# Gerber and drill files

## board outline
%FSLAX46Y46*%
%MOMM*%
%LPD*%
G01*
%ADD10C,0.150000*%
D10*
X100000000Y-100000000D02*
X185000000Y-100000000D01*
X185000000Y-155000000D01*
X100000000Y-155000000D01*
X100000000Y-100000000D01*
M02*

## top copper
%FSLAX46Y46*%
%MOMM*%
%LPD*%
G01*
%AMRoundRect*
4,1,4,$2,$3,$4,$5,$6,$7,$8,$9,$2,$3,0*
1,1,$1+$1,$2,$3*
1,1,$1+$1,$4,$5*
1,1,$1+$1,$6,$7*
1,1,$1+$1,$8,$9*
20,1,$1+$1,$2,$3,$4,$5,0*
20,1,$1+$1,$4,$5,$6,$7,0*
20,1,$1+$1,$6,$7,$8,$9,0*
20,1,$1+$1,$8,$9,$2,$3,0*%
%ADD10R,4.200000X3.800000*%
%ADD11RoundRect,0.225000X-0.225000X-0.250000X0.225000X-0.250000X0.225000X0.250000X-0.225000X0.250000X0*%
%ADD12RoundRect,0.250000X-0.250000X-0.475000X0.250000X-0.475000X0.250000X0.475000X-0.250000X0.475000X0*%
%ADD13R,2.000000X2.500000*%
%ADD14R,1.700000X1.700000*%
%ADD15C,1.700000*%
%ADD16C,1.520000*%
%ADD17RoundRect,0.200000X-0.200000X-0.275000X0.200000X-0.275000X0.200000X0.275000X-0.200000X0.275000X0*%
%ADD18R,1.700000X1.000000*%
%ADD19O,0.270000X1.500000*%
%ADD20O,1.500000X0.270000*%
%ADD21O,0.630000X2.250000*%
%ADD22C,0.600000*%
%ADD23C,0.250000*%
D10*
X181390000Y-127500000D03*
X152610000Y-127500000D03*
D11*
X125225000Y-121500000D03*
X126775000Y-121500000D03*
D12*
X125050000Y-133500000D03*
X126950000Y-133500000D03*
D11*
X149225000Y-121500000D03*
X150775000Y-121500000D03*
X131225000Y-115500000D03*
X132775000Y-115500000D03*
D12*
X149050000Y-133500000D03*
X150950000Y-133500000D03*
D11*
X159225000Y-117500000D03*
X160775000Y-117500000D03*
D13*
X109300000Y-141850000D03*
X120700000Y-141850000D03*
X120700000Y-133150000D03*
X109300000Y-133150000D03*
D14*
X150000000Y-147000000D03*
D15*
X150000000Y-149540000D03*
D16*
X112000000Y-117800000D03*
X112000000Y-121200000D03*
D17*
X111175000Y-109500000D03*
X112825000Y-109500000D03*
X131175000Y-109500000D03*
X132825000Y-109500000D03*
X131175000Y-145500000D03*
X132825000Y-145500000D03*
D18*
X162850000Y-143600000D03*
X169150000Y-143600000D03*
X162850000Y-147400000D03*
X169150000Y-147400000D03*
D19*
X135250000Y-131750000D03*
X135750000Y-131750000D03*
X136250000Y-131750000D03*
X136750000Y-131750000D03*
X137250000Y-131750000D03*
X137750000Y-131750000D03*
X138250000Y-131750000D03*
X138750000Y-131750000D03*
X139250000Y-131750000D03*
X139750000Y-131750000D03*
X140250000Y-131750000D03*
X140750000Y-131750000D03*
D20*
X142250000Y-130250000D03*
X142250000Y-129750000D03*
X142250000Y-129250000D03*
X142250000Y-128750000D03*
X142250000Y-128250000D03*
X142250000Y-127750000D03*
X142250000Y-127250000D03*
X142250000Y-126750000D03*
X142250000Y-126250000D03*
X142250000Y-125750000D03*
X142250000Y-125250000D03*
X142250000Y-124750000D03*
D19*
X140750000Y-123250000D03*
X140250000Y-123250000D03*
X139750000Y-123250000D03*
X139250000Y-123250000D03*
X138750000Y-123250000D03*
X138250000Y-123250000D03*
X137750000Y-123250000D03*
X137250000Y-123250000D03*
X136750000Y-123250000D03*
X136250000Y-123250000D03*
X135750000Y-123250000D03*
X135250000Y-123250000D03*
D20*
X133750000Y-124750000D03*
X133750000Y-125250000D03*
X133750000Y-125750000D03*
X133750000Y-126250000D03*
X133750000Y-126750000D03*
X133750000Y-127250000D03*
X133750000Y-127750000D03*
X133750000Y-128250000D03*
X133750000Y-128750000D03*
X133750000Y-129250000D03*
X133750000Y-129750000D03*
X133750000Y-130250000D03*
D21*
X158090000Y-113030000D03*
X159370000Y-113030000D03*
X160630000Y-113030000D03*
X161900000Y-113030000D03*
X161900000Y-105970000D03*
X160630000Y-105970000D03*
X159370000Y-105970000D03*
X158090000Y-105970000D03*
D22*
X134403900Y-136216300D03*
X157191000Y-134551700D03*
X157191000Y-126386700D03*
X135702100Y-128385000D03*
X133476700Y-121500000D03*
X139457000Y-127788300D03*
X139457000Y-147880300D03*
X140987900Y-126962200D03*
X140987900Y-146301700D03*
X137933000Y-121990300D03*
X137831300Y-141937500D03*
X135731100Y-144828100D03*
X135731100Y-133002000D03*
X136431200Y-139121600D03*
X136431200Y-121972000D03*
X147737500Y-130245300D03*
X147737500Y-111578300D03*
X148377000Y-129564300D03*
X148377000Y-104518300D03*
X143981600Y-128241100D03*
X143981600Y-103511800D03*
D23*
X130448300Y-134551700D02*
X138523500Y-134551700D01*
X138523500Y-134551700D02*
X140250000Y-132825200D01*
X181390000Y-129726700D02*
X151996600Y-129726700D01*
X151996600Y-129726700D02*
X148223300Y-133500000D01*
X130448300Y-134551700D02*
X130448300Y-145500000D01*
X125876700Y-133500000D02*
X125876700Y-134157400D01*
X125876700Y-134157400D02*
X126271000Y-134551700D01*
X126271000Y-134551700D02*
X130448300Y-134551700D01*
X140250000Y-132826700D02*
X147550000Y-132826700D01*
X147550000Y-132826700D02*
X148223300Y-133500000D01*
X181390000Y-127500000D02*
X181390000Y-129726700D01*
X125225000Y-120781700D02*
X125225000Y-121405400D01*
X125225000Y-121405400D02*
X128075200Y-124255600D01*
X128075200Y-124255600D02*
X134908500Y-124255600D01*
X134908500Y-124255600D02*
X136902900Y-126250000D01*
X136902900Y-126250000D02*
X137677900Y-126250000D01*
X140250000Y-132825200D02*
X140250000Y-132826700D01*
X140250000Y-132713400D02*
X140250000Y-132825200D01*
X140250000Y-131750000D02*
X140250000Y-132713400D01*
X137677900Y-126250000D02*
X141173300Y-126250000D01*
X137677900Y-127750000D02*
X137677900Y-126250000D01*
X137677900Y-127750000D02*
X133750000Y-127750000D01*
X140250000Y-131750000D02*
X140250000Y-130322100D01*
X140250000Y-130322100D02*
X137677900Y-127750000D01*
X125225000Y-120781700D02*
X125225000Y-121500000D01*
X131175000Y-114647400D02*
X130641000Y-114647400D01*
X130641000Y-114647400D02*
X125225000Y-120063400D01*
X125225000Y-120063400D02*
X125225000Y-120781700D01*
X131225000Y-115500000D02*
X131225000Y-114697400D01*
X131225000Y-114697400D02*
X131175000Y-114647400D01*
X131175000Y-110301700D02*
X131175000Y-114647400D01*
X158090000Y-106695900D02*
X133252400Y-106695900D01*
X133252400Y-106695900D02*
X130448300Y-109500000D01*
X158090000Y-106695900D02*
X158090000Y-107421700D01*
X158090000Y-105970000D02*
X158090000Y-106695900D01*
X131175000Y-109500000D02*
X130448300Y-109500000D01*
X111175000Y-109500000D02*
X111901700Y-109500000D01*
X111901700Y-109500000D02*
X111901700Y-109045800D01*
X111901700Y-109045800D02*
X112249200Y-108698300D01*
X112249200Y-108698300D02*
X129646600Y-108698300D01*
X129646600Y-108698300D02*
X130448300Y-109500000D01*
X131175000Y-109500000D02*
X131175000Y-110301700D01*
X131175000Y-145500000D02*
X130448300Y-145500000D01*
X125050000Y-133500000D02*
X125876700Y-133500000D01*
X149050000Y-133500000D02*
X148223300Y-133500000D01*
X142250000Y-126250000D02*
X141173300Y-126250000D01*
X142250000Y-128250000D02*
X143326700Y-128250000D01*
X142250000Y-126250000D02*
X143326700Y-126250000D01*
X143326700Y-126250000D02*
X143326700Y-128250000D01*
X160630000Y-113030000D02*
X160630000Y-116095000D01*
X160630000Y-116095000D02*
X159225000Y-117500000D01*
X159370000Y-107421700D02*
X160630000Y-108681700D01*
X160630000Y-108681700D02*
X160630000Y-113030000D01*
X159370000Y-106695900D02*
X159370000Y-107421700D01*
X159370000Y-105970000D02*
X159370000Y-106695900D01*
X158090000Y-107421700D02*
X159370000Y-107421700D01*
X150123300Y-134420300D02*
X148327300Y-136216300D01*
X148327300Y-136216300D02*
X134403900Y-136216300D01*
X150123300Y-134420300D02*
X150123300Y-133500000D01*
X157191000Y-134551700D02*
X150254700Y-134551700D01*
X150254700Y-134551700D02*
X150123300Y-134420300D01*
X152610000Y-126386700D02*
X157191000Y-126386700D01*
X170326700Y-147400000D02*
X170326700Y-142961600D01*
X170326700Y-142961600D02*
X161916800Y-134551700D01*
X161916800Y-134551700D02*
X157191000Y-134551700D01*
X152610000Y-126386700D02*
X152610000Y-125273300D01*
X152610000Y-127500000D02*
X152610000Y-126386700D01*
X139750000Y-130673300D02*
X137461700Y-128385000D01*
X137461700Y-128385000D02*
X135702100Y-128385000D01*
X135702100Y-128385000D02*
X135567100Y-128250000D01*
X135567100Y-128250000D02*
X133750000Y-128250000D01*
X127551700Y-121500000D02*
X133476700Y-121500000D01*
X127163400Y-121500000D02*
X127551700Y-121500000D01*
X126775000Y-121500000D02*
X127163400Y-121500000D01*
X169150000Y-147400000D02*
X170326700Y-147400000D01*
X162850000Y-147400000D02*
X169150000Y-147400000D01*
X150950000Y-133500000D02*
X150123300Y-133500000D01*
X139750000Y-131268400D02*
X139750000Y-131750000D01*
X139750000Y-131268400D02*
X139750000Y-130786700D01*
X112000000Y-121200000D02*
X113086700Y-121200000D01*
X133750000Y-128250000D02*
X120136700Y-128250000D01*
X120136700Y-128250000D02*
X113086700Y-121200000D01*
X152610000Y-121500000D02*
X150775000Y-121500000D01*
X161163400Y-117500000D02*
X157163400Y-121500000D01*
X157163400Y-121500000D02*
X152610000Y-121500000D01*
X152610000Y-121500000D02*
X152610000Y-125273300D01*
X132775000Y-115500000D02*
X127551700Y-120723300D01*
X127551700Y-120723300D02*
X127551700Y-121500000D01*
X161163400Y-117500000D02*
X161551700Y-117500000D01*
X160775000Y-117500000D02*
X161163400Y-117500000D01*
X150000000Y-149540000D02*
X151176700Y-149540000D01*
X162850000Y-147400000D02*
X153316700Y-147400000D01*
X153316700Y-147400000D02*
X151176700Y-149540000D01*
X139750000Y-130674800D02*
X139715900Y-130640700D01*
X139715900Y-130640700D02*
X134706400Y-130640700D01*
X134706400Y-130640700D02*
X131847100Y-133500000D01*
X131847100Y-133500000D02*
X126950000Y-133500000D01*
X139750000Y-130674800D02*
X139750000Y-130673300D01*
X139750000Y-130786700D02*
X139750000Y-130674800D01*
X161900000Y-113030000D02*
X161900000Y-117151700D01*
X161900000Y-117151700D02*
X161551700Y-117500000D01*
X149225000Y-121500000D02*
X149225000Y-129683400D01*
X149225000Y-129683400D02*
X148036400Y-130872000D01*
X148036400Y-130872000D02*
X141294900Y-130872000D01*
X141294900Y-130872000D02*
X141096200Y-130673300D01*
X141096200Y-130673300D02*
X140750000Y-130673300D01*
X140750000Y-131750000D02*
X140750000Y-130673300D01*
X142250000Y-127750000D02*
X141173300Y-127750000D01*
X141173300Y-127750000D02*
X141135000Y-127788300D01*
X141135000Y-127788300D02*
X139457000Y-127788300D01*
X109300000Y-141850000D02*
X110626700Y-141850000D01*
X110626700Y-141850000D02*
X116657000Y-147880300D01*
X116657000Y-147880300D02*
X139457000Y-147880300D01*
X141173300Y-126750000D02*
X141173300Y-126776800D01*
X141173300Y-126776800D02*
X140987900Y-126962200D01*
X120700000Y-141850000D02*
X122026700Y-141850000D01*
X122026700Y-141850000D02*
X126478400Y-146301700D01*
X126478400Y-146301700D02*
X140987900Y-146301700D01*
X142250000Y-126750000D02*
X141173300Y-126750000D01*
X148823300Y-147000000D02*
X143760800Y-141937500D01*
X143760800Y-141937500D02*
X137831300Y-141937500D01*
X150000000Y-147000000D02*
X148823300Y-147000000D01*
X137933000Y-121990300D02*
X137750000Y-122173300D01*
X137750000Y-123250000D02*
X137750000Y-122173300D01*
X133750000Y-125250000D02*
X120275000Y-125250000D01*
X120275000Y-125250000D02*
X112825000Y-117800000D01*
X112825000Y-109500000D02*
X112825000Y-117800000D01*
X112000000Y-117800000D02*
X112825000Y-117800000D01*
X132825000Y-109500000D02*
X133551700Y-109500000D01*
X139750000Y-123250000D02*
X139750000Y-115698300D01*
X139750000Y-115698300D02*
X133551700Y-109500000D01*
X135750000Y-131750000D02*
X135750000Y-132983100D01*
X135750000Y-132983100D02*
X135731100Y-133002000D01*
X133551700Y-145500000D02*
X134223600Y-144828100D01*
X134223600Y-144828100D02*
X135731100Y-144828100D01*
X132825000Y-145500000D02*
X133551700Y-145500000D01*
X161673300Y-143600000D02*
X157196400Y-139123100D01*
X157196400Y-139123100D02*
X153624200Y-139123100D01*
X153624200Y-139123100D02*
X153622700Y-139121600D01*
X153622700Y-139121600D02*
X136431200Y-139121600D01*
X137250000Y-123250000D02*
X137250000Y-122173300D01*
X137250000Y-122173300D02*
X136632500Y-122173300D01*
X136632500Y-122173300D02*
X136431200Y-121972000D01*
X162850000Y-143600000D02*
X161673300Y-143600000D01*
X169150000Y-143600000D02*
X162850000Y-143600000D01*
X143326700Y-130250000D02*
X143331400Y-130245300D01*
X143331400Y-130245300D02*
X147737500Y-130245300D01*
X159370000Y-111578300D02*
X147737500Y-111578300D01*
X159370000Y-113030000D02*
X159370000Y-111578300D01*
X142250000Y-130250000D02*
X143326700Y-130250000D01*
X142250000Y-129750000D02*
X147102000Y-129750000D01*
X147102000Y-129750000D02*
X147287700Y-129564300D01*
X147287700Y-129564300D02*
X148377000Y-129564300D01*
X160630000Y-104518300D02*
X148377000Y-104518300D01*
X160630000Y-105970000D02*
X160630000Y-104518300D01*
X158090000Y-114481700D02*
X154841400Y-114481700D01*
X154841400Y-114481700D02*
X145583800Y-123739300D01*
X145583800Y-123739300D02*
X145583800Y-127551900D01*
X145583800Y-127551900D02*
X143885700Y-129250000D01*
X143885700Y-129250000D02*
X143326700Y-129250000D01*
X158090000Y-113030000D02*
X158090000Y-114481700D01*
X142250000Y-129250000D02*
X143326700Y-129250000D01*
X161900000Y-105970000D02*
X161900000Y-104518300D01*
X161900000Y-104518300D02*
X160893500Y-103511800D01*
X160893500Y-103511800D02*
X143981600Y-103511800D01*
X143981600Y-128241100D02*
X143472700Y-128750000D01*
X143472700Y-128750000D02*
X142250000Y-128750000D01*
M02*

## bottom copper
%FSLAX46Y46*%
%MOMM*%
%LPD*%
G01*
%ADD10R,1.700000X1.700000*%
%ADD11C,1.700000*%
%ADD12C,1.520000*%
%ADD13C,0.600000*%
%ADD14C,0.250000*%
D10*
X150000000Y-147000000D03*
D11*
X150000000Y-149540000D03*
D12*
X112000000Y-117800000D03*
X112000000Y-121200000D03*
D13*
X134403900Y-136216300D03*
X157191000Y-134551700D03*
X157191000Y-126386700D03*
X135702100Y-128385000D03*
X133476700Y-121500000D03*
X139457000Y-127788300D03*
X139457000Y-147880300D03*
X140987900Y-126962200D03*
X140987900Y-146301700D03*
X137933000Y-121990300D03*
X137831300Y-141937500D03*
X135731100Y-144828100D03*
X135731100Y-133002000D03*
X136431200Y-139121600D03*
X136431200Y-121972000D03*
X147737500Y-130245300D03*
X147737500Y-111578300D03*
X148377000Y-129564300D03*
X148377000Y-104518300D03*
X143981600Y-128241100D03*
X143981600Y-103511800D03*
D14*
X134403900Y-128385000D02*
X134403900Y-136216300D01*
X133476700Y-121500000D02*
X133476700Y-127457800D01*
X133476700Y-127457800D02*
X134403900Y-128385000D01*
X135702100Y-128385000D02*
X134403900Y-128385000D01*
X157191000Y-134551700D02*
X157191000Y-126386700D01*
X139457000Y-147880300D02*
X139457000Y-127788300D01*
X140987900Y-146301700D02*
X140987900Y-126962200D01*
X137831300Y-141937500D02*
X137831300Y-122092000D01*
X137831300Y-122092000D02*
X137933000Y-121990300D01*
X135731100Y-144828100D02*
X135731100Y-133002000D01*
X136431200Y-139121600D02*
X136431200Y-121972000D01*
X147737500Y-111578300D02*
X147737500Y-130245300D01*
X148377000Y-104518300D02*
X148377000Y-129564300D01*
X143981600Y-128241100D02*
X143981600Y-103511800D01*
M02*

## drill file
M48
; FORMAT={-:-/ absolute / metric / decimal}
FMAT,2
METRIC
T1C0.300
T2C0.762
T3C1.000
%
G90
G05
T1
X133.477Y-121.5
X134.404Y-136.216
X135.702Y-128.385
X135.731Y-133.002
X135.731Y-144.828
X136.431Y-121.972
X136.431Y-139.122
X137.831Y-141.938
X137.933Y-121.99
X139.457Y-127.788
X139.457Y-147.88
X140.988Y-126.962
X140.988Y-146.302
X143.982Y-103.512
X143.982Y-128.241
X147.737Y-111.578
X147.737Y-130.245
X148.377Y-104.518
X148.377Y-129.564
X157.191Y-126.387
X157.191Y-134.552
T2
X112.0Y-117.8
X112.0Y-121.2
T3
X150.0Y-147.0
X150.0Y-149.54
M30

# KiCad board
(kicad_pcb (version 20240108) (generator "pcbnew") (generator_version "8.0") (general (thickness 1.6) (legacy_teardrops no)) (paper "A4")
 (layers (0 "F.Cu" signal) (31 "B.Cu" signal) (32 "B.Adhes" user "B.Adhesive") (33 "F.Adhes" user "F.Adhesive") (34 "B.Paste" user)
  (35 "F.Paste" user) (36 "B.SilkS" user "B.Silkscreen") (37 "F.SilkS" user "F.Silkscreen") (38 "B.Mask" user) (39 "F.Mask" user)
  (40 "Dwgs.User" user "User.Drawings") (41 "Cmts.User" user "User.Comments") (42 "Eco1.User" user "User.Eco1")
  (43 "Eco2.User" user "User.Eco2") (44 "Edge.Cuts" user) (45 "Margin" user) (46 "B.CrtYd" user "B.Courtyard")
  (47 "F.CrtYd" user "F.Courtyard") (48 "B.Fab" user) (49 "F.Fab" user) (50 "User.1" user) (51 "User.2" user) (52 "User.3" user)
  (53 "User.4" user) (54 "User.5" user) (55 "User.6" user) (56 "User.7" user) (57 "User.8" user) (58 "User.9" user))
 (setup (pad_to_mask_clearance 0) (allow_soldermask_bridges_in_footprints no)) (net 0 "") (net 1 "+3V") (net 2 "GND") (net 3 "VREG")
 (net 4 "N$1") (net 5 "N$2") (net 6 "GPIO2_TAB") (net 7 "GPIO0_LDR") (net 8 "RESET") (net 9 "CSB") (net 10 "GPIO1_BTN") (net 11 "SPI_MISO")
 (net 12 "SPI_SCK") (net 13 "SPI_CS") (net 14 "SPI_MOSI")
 (gr_rect (start 100.0 100.0) (end 185.0 155.0) (stroke (width 0.15) (type default)) (fill none) (layer "Edge.Cuts"))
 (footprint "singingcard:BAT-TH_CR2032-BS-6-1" (layer "F.Cu") (at 167.0 127.5 0)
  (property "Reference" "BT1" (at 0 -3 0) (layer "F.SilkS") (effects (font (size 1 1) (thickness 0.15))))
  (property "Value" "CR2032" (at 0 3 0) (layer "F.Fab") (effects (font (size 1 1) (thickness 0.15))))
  (pad "1" smd rect (at 14.39 0) (size 4.2 3.8) (layers "F.Cu" "F.Mask" "F.Paste") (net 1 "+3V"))
  (pad "2" smd rect (at -14.39 0) (size 4.2 3.8) (layers "F.Cu" "F.Mask" "F.Paste") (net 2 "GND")))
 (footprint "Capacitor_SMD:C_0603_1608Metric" (layer "F.Cu") (at 126.0 121.5 0)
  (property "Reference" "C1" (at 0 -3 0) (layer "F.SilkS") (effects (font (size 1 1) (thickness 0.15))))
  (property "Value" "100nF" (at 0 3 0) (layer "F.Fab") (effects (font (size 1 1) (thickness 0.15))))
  (pad "1" smd roundrect (at -0.775 0) (size 0.9 0.95) (layers "F.Cu" "F.Mask" "F.Paste") (roundrect_rratio 0.25) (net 1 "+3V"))
  (pad "2" smd roundrect (at 0.775 0) (size 0.9 0.95) (layers "F.Cu" "F.Mask" "F.Paste") (roundrect_rratio 0.25) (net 2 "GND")))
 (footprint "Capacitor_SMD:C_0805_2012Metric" (layer "F.Cu") (at 126.0 133.5 0)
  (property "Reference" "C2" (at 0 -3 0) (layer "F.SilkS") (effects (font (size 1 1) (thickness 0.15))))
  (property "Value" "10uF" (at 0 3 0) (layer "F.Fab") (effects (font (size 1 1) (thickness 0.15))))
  (pad "1" smd roundrect (at -0.95 0) (size 1 1.45) (layers "F.Cu" "F.Mask" "F.Paste") (roundrect_rratio 0.25) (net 1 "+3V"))
  (pad "2" smd roundrect (at 0.95 0) (size 1 1.45) (layers "F.Cu" "F.Mask" "F.Paste") (roundrect_rratio 0.25) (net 2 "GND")))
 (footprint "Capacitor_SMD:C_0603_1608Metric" (layer "F.Cu") (at 150.0 121.5 0)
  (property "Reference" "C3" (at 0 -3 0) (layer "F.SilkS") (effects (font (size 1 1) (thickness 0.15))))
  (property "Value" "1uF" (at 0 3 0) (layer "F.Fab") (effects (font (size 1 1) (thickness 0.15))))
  (pad "1" smd roundrect (at -0.775 0) (size 0.9 0.95) (layers "F.Cu" "F.Mask" "F.Paste") (roundrect_rratio 0.25) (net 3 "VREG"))
  (pad "2" smd roundrect (at 0.775 0) (size 0.9 0.95) (layers "F.Cu" "F.Mask" "F.Paste") (roundrect_rratio 0.25) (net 2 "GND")))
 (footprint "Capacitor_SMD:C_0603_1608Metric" (layer "F.Cu") (at 132.0 115.5 0)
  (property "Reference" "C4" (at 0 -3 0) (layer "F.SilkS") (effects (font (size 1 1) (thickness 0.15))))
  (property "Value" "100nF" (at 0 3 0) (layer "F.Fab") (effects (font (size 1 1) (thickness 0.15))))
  (pad "1" smd roundrect (at -0.775 0) (size 0.9 0.95) (layers "F.Cu" "F.Mask" "F.Paste") (roundrect_rratio 0.25) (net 1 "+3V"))
  (pad "2" smd roundrect (at 0.775 0) (size 0.9 0.95) (layers "F.Cu" "F.Mask" "F.Paste") (roundrect_rratio 0.25) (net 2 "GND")))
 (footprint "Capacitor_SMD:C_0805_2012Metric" (layer "F.Cu") (at 150.0 133.5 0)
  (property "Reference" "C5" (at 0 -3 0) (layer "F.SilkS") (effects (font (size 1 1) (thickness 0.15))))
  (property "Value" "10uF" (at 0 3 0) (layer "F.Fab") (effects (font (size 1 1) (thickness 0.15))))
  (pad "1" smd roundrect (at -0.95 0) (size 1 1.45) (layers "F.Cu" "F.Mask" "F.Paste") (roundrect_rratio 0.25) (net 1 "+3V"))
  (pad "2" smd roundrect (at 0.95 0) (size 1 1.45) (layers "F.Cu" "F.Mask" "F.Paste") (roundrect_rratio 0.25) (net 2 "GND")))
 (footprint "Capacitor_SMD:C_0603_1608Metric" (layer "F.Cu") (at 160.0 117.5 0)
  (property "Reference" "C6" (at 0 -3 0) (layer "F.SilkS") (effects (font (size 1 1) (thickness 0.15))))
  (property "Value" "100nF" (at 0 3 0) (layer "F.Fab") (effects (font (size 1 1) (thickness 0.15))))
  (pad "1" smd roundrect (at -0.775 0) (size 0.9 0.95) (layers "F.Cu" "F.Mask" "F.Paste") (roundrect_rratio 0.25) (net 1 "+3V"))
  (pad "2" smd roundrect (at 0.775 0) (size 0.9 0.95) (layers "F.Cu" "F.Mask" "F.Paste") (roundrect_rratio 0.25) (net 2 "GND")))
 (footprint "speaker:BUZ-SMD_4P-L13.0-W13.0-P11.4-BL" (layer "F.Cu") (at 115.0 137.5 0)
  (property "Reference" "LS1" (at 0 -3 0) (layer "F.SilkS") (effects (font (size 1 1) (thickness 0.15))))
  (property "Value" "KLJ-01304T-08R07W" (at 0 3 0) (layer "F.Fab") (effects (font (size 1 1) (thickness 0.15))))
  (pad "1" smd rect (at -5.7 4.35) (size 2 2.5) (layers "F.Cu" "F.Mask" "F.Paste") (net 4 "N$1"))
  (pad "2" smd rect (at 5.7 4.35) (size 2 2.5) (layers "F.Cu" "F.Mask" "F.Paste") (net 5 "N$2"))
  (pad "3" smd rect (at 5.7 -4.35) (size 2 2.5) (layers "F.Cu" "F.Mask" "F.Paste"))
  (pad "4" smd rect (at -5.7 -4.35) (size 2 2.5) (layers "F.Cu" "F.Mask" "F.Paste")))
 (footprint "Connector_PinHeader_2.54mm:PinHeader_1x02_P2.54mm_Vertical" (layer "F.Cu") (at 150.0 147.0 0)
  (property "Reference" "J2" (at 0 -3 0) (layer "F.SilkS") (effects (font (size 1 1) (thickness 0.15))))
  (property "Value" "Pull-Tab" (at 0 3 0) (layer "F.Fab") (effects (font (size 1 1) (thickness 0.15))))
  (pad "1" thru_hole rect (at 0 0) (size 1.7 1.7) (drill 1) (layers "*.Cu" "*.Mask") (remove_unused_layers no) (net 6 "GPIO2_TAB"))
  (pad "2" thru_hole circle (at 0 2.54) (size 1.7 1.7) (drill 1) (layers "*.Cu" "*.Mask") (remove_unused_layers no) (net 2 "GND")))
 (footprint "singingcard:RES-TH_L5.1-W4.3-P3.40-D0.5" (layer "F.Cu") (at 112.0 119.5 0)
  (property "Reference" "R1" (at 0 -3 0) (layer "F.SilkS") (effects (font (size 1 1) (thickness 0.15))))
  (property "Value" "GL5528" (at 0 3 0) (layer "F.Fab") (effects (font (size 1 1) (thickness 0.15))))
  (pad "1" thru_hole circle (at 0 -1.7 270) (size 1.52 1.52) (drill 0.762) (layers "*.Cu" "*.Mask") (remove_unused_layers no)
   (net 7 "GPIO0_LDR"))
  (pad "2" thru_hole circle (at 0 1.7 270) (size 1.52 1.52) (drill 0.762) (layers "*.Cu" "*.Mask") (remove_unused_layers no) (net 2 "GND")))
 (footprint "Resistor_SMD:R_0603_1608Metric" (layer "F.Cu") (at 112.0 109.5 0)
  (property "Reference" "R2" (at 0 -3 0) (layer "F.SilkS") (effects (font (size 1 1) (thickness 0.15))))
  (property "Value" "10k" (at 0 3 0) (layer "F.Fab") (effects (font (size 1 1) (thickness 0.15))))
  (pad "1" smd roundrect (at -0.825 0) (size 0.8 0.95) (layers "F.Cu" "F.Mask" "F.Paste") (roundrect_rratio 0.25) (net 1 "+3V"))
  (pad "2" smd roundrect (at 0.825 0) (size 0.8 0.95) (layers "F.Cu" "F.Mask" "F.Paste") (roundrect_rratio 0.25) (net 7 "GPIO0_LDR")))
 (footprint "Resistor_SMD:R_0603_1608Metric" (layer "F.Cu") (at 132.0 109.5 0)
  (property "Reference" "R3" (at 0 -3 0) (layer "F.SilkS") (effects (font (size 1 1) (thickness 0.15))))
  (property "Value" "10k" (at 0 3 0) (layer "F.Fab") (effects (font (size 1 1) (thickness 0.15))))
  (pad "1" smd roundrect (at -0.825 0) (size 0.8 0.95) (layers "F.Cu" "F.Mask" "F.Paste") (roundrect_rratio 0.25) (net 1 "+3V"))
  (pad "2" smd roundrect (at 0.825 0) (size 0.8 0.95) (layers "F.Cu" "F.Mask" "F.Paste") (roundrect_rratio 0.25) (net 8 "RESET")))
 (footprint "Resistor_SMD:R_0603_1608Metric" (layer "F.Cu") (at 132.0 145.5 0)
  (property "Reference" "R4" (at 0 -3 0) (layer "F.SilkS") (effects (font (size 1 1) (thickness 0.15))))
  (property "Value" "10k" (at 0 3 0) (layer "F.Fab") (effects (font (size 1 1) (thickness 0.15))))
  (pad "1" smd roundrect (at -0.825 0) (size 0.8 0.95) (layers "F.Cu" "F.Mask" "F.Paste") (roundrect_rratio 0.25) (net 1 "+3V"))
  (pad "2" smd roundrect (at 0.825 0) (size 0.8 0.95) (layers "F.Cu" "F.Mask" "F.Paste") (roundrect_rratio 0.25) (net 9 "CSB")))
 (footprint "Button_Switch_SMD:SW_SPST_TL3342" (layer "F.Cu") (at 166.0 145.5 0)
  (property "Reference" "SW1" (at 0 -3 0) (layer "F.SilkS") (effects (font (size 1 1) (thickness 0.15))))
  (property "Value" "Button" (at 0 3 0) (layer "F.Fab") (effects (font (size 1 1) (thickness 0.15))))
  (pad "1" smd rect (at -3.15 -1.9) (size 1.7 1) (layers "F.Cu" "F.Mask" "F.Paste") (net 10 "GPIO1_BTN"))
  (pad "1" smd rect (at 3.15 -1.9) (size 1.7 1) (layers "F.Cu" "F.Mask" "F.Paste") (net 10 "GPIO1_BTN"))
  (pad "2" smd rect (at -3.15 1.9) (size 1.7 1) (layers "F.Cu" "F.Mask" "F.Paste") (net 2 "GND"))
  (pad "2" smd rect (at 3.15 1.9) (size 1.7 1) (layers "F.Cu" "F.Mask" "F.Paste") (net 2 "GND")))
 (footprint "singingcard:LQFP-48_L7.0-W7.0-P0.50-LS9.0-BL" (layer "F.Cu") (at 138.0 127.5 0)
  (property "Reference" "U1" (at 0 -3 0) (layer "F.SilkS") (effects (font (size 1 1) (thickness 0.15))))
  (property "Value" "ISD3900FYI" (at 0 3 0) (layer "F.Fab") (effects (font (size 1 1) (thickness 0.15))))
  (pad "1" smd oval (at -2.75 4.25) (size 0.27 1.5) (layers "F.Cu" "F.Mask" "F.Paste"))
  (pad "2" smd oval (at -2.25 4.25) (size 0.27 1.5) (layers "F.Cu" "F.Mask" "F.Paste") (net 9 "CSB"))
  (pad "3" smd oval (at -1.75 4.25) (size 0.27 1.5) (layers "F.Cu" "F.Mask" "F.Paste"))
  (pad "4" smd oval (at -1.25 4.25) (size 0.27 1.5) (layers "F.Cu" "F.Mask" "F.Paste"))
  (pad "5" smd oval (at -0.75 4.25) (size 0.27 1.5) (layers "F.Cu" "F.Mask" "F.Paste"))
  (pad "6" smd oval (at -0.25 4.25) (size 0.27 1.5) (layers "F.Cu" "F.Mask" "F.Paste"))
  (pad "7" smd oval (at 0.25 4.25) (size 0.27 1.5) (layers "F.Cu" "F.Mask" "F.Paste"))
  (pad "8" smd oval (at 0.75 4.25) (size 0.27 1.5) (layers "F.Cu" "F.Mask" "F.Paste"))
  (pad "9" smd oval (at 1.25 4.25) (size 0.27 1.5) (layers "F.Cu" "F.Mask" "F.Paste"))
  (pad "10" smd oval (at 1.75 4.25) (size 0.27 1.5) (layers "F.Cu" "F.Mask" "F.Paste") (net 2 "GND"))
  (pad "11" smd oval (at 2.25 4.25) (size 0.27 1.5) (layers "F.Cu" "F.Mask" "F.Paste") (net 1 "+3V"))
  (pad "12" smd oval (at 2.75 4.25) (size 0.27 1.5) (layers "F.Cu" "F.Mask" "F.Paste") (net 3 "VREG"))
  (pad "13" smd oval (at 4.25 2.75) (size 1.5 0.27) (layers "F.Cu" "F.Mask" "F.Paste") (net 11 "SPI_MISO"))
  (pad "14" smd oval (at 4.25 2.25) (size 1.5 0.27) (layers "F.Cu" "F.Mask" "F.Paste") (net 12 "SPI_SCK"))
  (pad "15" smd oval (at 4.25 1.75) (size 1.5 0.27) (layers "F.Cu" "F.Mask" "F.Paste") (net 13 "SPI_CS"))
  (pad "16" smd oval (at 4.25 1.25) (size 1.5 0.27) (layers "F.Cu" "F.Mask" "F.Paste") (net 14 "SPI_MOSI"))
  (pad "17" smd oval (at 4.25 0.75) (size 1.5 0.27) (layers "F.Cu" "F.Mask" "F.Paste") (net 1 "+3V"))
  (pad "18" smd oval (at 4.25 0.25) (size 1.5 0.27) (layers "F.Cu" "F.Mask" "F.Paste") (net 4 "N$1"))
  (pad "19" smd oval (at 4.25 -0.25) (size 1.5 0.27) (layers "F.Cu" "F.Mask" "F.Paste"))
  (pad "20" smd oval (at 4.25 -0.75) (size 1.5 0.27) (layers "F.Cu" "F.Mask" "F.Paste") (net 5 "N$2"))
  (pad "21" smd oval (at 4.25 -1.25) (size 1.5 0.27) (layers "F.Cu" "F.Mask" "F.Paste") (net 1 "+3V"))
  (pad "22" smd oval (at 4.25 -1.75) (size 1.5 0.27) (layers "F.Cu" "F.Mask" "F.Paste"))
  (pad "23" smd oval (at 4.25 -2.25) (size 1.5 0.27) (layers "F.Cu" "F.Mask" "F.Paste"))
  (pad "24" smd oval (at 4.25 -2.75) (size 1.5 0.27) (layers "F.Cu" "F.Mask" "F.Paste"))
  (pad "25" smd oval (at 2.75 -4.25) (size 0.27 1.5) (layers "F.Cu" "F.Mask" "F.Paste"))
  (pad "26" smd oval (at 2.25 -4.25) (size 0.27 1.5) (layers "F.Cu" "F.Mask" "F.Paste"))
  (pad "27" smd oval (at 1.75 -4.25) (size 0.27 1.5) (layers "F.Cu" "F.Mask" "F.Paste") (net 8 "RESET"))
  (pad "28" smd oval (at 1.25 -4.25) (size 0.27 1.5) (layers "F.Cu" "F.Mask" "F.Paste"))
  (pad "29" smd oval (at 0.75 -4.25) (size 0.27 1.5) (layers "F.Cu" "F.Mask" "F.Paste"))
  (pad "30" smd oval (at 0.25 -4.25) (size 0.27 1.5) (layers "F.Cu" "F.Mask" "F.Paste"))
  (pad "31" smd oval (at -0.25 -4.25) (size 0.27 1.5) (layers "F.Cu" "F.Mask" "F.Paste") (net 6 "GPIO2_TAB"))
  (pad "32" smd oval (at -0.75 -4.25) (size 0.27 1.5) (layers "F.Cu" "F.Mask" "F.Paste") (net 10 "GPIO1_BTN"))
  (pad "33" smd oval (at -1.25 -4.25) (size 0.27 1.5) (layers "F.Cu" "F.Mask" "F.Paste"))
  (pad "34" smd oval (at -1.75 -4.25) (size 0.27 1.5) (layers "F.Cu" "F.Mask" "F.Paste"))
  (pad "35" smd oval (at -2.25 -4.25) (size 0.27 1.5) (layers "F.Cu" "F.Mask" "F.Paste"))
  (pad "36" smd oval (at -2.75 -4.25) (size 0.27 1.5) (layers "F.Cu" "F.Mask" "F.Paste"))
  (pad "37" smd oval (at -4.25 -2.75) (size 1.5 0.27) (layers "F.Cu" "F.Mask" "F.Paste"))
  (pad "38" smd oval (at -4.25 -2.25) (size 1.5 0.27) (layers "F.Cu" "F.Mask" "F.Paste") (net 7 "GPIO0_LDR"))
  (pad "39" smd oval (at -4.25 -1.75) (size 1.5 0.27) (layers "F.Cu" "F.Mask" "F.Paste"))
  (pad "40" smd oval (at -4.25 -1.25) (size 1.5 0.27) (layers "F.Cu" "F.Mask" "F.Paste"))
  (pad "41" smd oval (at -4.25 -0.75) (size 1.5 0.27) (layers "F.Cu" "F.Mask" "F.Paste"))
  (pad "42" smd oval (at -4.25 -0.25) (size 1.5 0.27) (layers "F.Cu" "F.Mask" "F.Paste"))
  (pad "43" smd oval (at -4.25 0.25) (size 1.5 0.27) (layers "F.Cu" "F.Mask" "F.Paste") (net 1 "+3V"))
  (pad "44" smd oval (at -4.25 0.75) (size 1.5 0.27) (layers "F.Cu" "F.Mask" "F.Paste") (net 2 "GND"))
  (pad "45" smd oval (at -4.25 1.25) (size 1.5 0.27) (layers "F.Cu" "F.Mask" "F.Paste"))
  (pad "46" smd oval (at -4.25 1.75) (size 1.5 0.27) (layers "F.Cu" "F.Mask" "F.Paste"))
  (pad "47" smd oval (at -4.25 2.25) (size 1.5 0.27) (layers "F.Cu" "F.Mask" "F.Paste"))
  (pad "48" smd oval (at -4.25 2.75) (size 1.5 0.27) (layers "F.Cu" "F.Mask" "F.Paste")))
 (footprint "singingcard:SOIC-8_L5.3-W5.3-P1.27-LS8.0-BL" (layer "F.Cu") (at 160.0 109.5 0)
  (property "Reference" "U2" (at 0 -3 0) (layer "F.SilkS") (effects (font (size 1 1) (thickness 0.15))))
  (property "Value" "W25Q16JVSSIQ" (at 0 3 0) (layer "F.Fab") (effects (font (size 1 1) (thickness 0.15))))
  (pad "1" smd oval (at -1.91 3.53) (size 0.63 2.25) (layers "F.Cu" "F.Mask" "F.Paste") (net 13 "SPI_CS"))
  (pad "2" smd oval (at -0.63 3.53) (size 0.63 2.25) (layers "F.Cu" "F.Mask" "F.Paste") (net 11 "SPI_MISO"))
  (pad "3" smd oval (at 0.63 3.53) (size 0.63 2.25) (layers "F.Cu" "F.Mask" "F.Paste") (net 1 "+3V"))
  (pad "4" smd oval (at 1.9 3.53) (size 0.63 2.25) (layers "F.Cu" "F.Mask" "F.Paste") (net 2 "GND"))
  (pad "5" smd oval (at 1.9 -3.53) (size 0.63 2.25) (layers "F.Cu" "F.Mask" "F.Paste") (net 14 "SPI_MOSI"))
  (pad "6" smd oval (at 0.63 -3.53) (size 0.63 2.25) (layers "F.Cu" "F.Mask" "F.Paste") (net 12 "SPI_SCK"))
  (pad "7" smd oval (at -0.63 -3.53) (size 0.63 2.25) (layers "F.Cu" "F.Mask" "F.Paste") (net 1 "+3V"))
  (pad "8" smd oval (at -1.91 -3.53) (size 0.63 2.25) (layers "F.Cu" "F.Mask" "F.Paste") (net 1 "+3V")))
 (segment (start 130.4483 134.5517) (end 138.5235 134.5517) (width 0.2500) (layer "F.Cu") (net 1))
 (segment (start 138.5235 134.5517) (end 140.2500 132.8252) (width 0.2500) (layer "F.Cu") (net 1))
 (segment (start 181.3900 129.7267) (end 151.9966 129.7267) (width 0.2500) (layer "F.Cu") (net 1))
 (segment (start 151.9966 129.7267) (end 148.2233 133.5000) (width 0.2500) (layer "F.Cu") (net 1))
 (segment (start 130.4483 134.5517) (end 130.4483 145.5000) (width 0.2500) (layer "F.Cu") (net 1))
 (segment (start 125.8767 133.5000) (end 125.8767 134.1574) (width 0.2500) (layer "F.Cu") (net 1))
 (segment (start 125.8767 134.1574) (end 126.2710 134.5517) (width 0.2500) (layer "F.Cu") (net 1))
 (segment (start 126.2710 134.5517) (end 130.4483 134.5517) (width 0.2500) (layer "F.Cu") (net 1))
 (segment (start 140.2500 132.8267) (end 147.5500 132.8267) (width 0.2500) (layer "F.Cu") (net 1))
 (segment (start 147.5500 132.8267) (end 148.2233 133.5000) (width 0.2500) (layer "F.Cu") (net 1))
 (segment (start 181.3900 127.5000) (end 181.3900 129.7267) (width 0.2500) (layer "F.Cu") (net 1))
 (segment (start 125.2250 120.7817) (end 125.2250 121.4054) (width 0.2500) (layer "F.Cu") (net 1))
 (segment (start 125.2250 121.4054) (end 128.0752 124.2556) (width 0.2500) (layer "F.Cu") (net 1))
 (segment (start 128.0752 124.2556) (end 134.9085 124.2556) (width 0.2500) (layer "F.Cu") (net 1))
 (segment (start 134.9085 124.2556) (end 136.9029 126.2500) (width 0.2500) (layer "F.Cu") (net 1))
 (segment (start 136.9029 126.2500) (end 137.6779 126.2500) (width 0.2500) (layer "F.Cu") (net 1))
 (segment (start 140.2500 132.8252) (end 140.2500 132.8267) (width 0.2500) (layer "F.Cu") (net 1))
 (segment (start 140.2500 132.7134) (end 140.2500 132.8252) (width 0.2500) (layer "F.Cu") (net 1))
 (segment (start 140.2500 131.7500) (end 140.2500 132.7134) (width 0.2500) (layer "F.Cu") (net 1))
 (segment (start 137.6779 126.2500) (end 141.1733 126.2500) (width 0.2500) (layer "F.Cu") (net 1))
 (segment (start 137.6779 127.7500) (end 137.6779 126.2500) (width 0.2500) (layer "F.Cu") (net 1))
 (segment (start 137.6779 127.7500) (end 133.7500 127.7500) (width 0.2500) (layer "F.Cu") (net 1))
 (segment (start 140.2500 131.7500) (end 140.2500 130.3221) (width 0.2500) (layer "F.Cu") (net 1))
 (segment (start 140.2500 130.3221) (end 137.6779 127.7500) (width 0.2500) (layer "F.Cu") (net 1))
 (segment (start 125.2250 120.7817) (end 125.2250 121.5000) (width 0.2500) (layer "F.Cu") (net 1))
 (segment (start 131.1750 114.6474) (end 130.6410 114.6474) (width 0.2500) (layer "F.Cu") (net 1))
 (segment (start 130.6410 114.6474) (end 125.2250 120.0634) (width 0.2500) (layer "F.Cu") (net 1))
 (segment (start 125.2250 120.0634) (end 125.2250 120.7817) (width 0.2500) (layer "F.Cu") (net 1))
 (segment (start 131.2250 115.5000) (end 131.2250 114.6974) (width 0.2500) (layer "F.Cu") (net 1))
 (segment (start 131.2250 114.6974) (end 131.1750 114.6474) (width 0.2500) (layer "F.Cu") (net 1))
 (segment (start 131.1750 110.3017) (end 131.1750 114.6474) (width 0.2500) (layer "F.Cu") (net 1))
 (segment (start 158.0900 106.6959) (end 133.2524 106.6959) (width 0.2500) (layer "F.Cu") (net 1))
 (segment (start 133.2524 106.6959) (end 130.4483 109.5000) (width 0.2500) (layer "F.Cu") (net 1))
 (segment (start 158.0900 106.6959) (end 158.0900 107.4217) (width 0.2500) (layer "F.Cu") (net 1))
 (segment (start 158.0900 105.9700) (end 158.0900 106.6959) (width 0.2500) (layer "F.Cu") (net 1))
 (segment (start 131.1750 109.5000) (end 130.4483 109.5000) (width 0.2500) (layer "F.Cu") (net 1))
 (segment (start 111.1750 109.5000) (end 111.9017 109.5000) (width 0.2500) (layer "F.Cu") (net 1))
 (segment (start 111.9017 109.5000) (end 111.9017 109.0458) (width 0.2500) (layer "F.Cu") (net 1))
 (segment (start 111.9017 109.0458) (end 112.2492 108.6983) (width 0.2500) (layer "F.Cu") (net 1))
 (segment (start 112.2492 108.6983) (end 129.6466 108.6983) (width 0.2500) (layer "F.Cu") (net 1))
 (segment (start 129.6466 108.6983) (end 130.4483 109.5000) (width 0.2500) (layer "F.Cu") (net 1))
 (segment (start 131.1750 109.5000) (end 131.1750 110.3017) (width 0.2500) (layer "F.Cu") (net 1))
 (segment (start 131.1750 145.5000) (end 130.4483 145.5000) (width 0.2500) (layer "F.Cu") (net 1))
 (segment (start 125.0500 133.5000) (end 125.8767 133.5000) (width 0.2500) (layer "F.Cu") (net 1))
 (segment (start 149.0500 133.5000) (end 148.2233 133.5000) (width 0.2500) (layer "F.Cu") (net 1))
 (segment (start 142.2500 126.2500) (end 141.1733 126.2500) (width 0.2500) (layer "F.Cu") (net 1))
 (segment (start 142.2500 128.2500) (end 143.3267 128.2500) (width 0.2500) (layer "F.Cu") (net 1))
 (segment (start 142.2500 126.2500) (end 143.3267 126.2500) (width 0.2500) (layer "F.Cu") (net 1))
 (segment (start 143.3267 126.2500) (end 143.3267 128.2500) (width 0.2500) (layer "F.Cu") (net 1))
 (segment (start 160.6300 113.0300) (end 160.6300 116.0950) (width 0.2500) (layer "F.Cu") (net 1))
 (segment (start 160.6300 116.0950) (end 159.2250 117.5000) (width 0.2500) (layer "F.Cu") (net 1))
 (segment (start 159.3700 107.4217) (end 160.6300 108.6817) (width 0.2500) (layer "F.Cu") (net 1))
 (segment (start 160.6300 108.6817) (end 160.6300 113.0300) (width 0.2500) (layer "F.Cu") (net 1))
 (segment (start 159.3700 106.6959) (end 159.3700 107.4217) (width 0.2500) (layer "F.Cu") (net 1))
 (segment (start 159.3700 105.9700) (end 159.3700 106.6959) (width 0.2500) (layer "F.Cu") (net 1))
 (segment (start 158.0900 107.4217) (end 159.3700 107.4217) (width 0.2500) (layer "F.Cu") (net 1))
 (segment (start 134.4039 128.3850) (end 134.4039 136.2163) (width 0.2500) (layer "B.Cu") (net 2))
 (segment (start 133.4767 121.5000) (end 133.4767 127.4578) (width 0.2500) (layer "B.Cu") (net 2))
 (segment (start 133.4767 127.4578) (end 134.4039 128.3850) (width 0.2500) (layer "B.Cu") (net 2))
 (segment (start 135.7021 128.3850) (end 134.4039 128.3850) (width 0.2500) (layer "B.Cu") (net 2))
 (segment (start 150.1233 134.4203) (end 148.3273 136.2163) (width 0.2500) (layer "F.Cu") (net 2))
 (segment (start 148.3273 136.2163) (end 134.4039 136.2163) (width 0.2500) (layer "F.Cu") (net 2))
 (segment (start 150.1233 134.4203) (end 150.1233 133.5000) (width 0.2500) (layer "F.Cu") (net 2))
 (segment (start 157.1910 134.5517) (end 150.2547 134.5517) (width 0.2500) (layer "F.Cu") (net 2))
 (segment (start 150.2547 134.5517) (end 150.1233 134.4203) (width 0.2500) (layer "F.Cu") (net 2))
 (segment (start 152.6100 126.3867) (end 157.1910 126.3867) (width 0.2500) (layer "F.Cu") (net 2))
 (segment (start 157.1910 134.5517) (end 157.1910 126.3867) (width 0.2500) (layer "B.Cu") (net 2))
 (segment (start 170.3267 147.4000) (end 170.3267 142.9616) (width 0.2500) (layer "F.Cu") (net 2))
 (segment (start 170.3267 142.9616) (end 161.9168 134.5517) (width 0.2500) (layer "F.Cu") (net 2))
 (segment (start 161.9168 134.5517) (end 157.1910 134.5517) (width 0.2500) (layer "F.Cu") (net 2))
 (segment (start 152.6100 126.3867) (end 152.6100 125.2733) (width 0.2500) (layer "F.Cu") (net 2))
 (segment (start 152.6100 127.5000) (end 152.6100 126.3867) (width 0.2500) (layer "F.Cu") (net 2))
 (segment (start 139.7500 130.6733) (end 137.4617 128.3850) (width 0.2500) (layer "F.Cu") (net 2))
 (segment (start 137.4617 128.3850) (end 135.7021 128.3850) (width 0.2500) (layer "F.Cu") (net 2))
 (segment (start 135.7021 128.3850) (end 135.5671 128.2500) (width 0.2500) (layer "F.Cu") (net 2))
 (segment (start 135.5671 128.2500) (end 133.7500 128.2500) (width 0.2500) (layer "F.Cu") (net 2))
 (segment (start 127.5517 121.5000) (end 133.4767 121.5000) (width 0.2500) (layer "F.Cu") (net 2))
 (segment (start 127.1634 121.5000) (end 127.5517 121.5000) (width 0.2500) (layer "F.Cu") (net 2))
 (segment (start 126.7750 121.5000) (end 127.1634 121.5000) (width 0.2500) (layer "F.Cu") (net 2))
 (segment (start 169.1500 147.4000) (end 170.3267 147.4000) (width 0.2500) (layer "F.Cu") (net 2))
 (segment (start 162.8500 147.4000) (end 169.1500 147.4000) (width 0.2500) (layer "F.Cu") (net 2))
 (segment (start 150.9500 133.5000) (end 150.1233 133.5000) (width 0.2500) (layer "F.Cu") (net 2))
 (segment (start 139.7500 131.2684) (end 139.7500 131.7500) (width 0.2500) (layer "F.Cu") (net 2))
 (segment (start 139.7500 131.2684) (end 139.7500 130.7867) (width 0.2500) (layer "F.Cu") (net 2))
 (segment (start 112.0000 121.2000) (end 113.0867 121.2000) (width 0.2500) (layer "F.Cu") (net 2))
 (segment (start 133.7500 128.2500) (end 120.1367 128.2500) (width 0.2500) (layer "F.Cu") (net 2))
 (segment (start 120.1367 128.2500) (end 113.0867 121.2000) (width 0.2500) (layer "F.Cu") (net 2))
 (segment (start 152.6100 121.5000) (end 150.7750 121.5000) (width 0.2500) (layer "F.Cu") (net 2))
 (segment (start 161.1634 117.5000) (end 157.1634 121.5000) (width 0.2500) (layer "F.Cu") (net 2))
 (segment (start 157.1634 121.5000) (end 152.6100 121.5000) (width 0.2500) (layer "F.Cu") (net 2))
 (segment (start 152.6100 121.5000) (end 152.6100 125.2733) (width 0.2500) (layer "F.Cu") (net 2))
 (segment (start 132.7750 115.5000) (end 127.5517 120.7233) (width 0.2500) (layer "F.Cu") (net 2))
 (segment (start 127.5517 120.7233) (end 127.5517 121.5000) (width 0.2500) (layer "F.Cu") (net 2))
 (segment (start 161.1634 117.5000) (end 161.5517 117.5000) (width 0.2500) (layer "F.Cu") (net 2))
 (segment (start 160.7750 117.5000) (end 161.1634 117.5000) (width 0.2500) (layer "F.Cu") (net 2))
 (segment (start 150.0000 149.5400) (end 151.1767 149.5400) (width 0.2500) (layer "F.Cu") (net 2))
 (segment (start 162.8500 147.4000) (end 153.3167 147.4000) (width 0.2500) (layer "F.Cu") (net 2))
 (segment (start 153.3167 147.4000) (end 151.1767 149.5400) (width 0.2500) (layer "F.Cu") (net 2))
 (segment (start 139.7500 130.6748) (end 139.7159 130.6407) (width 0.2500) (layer "F.Cu") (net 2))
 (segment (start 139.7159 130.6407) (end 134.7064 130.6407) (width 0.2500) (layer "F.Cu") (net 2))
 (segment (start 134.7064 130.6407) (end 131.8471 133.5000) (width 0.2500) (layer "F.Cu") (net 2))
 (segment (start 131.8471 133.5000) (end 126.9500 133.5000) (width 0.2500) (layer "F.Cu") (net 2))
 (segment (start 139.7500 130.6748) (end 139.7500 130.6733) (width 0.2500) (layer "F.Cu") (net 2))
 (segment (start 139.7500 130.7867) (end 139.7500 130.6748) (width 0.2500) (layer "F.Cu") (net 2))
 (segment (start 161.9000 113.0300) (end 161.9000 117.1517) (width 0.2500) (layer "F.Cu") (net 2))
 (segment (start 161.9000 117.1517) (end 161.5517 117.5000) (width 0.2500) (layer "F.Cu") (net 2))
 (segment (start 149.2250 121.5000) (end 149.2250 129.6834) (width 0.2500) (layer "F.Cu") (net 3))
 (segment (start 149.2250 129.6834) (end 148.0364 130.8720) (width 0.2500) (layer "F.Cu") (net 3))
 (segment (start 148.0364 130.8720) (end 141.2949 130.8720) (width 0.2500) (layer "F.Cu") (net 3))
 (segment (start 141.2949 130.8720) (end 141.0962 130.6733) (width 0.2500) (layer "F.Cu") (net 3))
 (segment (start 141.0962 130.6733) (end 140.7500 130.6733) (width 0.2500) (layer "F.Cu") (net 3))
 (segment (start 140.7500 131.7500) (end 140.7500 130.6733) (width 0.2500) (layer "F.Cu") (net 3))
 (segment (start 142.2500 127.7500) (end 141.1733 127.7500) (width 0.2500) (layer "F.Cu") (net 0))
 (segment (start 141.1733 127.7500) (end 141.1350 127.7883) (width 0.2500) (layer "F.Cu") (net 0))
 (segment (start 141.1350 127.7883) (end 139.4570 127.7883) (width 0.2500) (layer "F.Cu") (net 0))
 (segment (start 139.4570 147.8803) (end 139.4570 127.7883) (width 0.2500) (layer "B.Cu") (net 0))
 (segment (start 109.3000 141.8500) (end 110.6267 141.8500) (width 0.2500) (layer "F.Cu") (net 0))
 (segment (start 110.6267 141.8500) (end 116.6570 147.8803) (width 0.2500) (layer "F.Cu") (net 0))
 (segment (start 116.6570 147.8803) (end 139.4570 147.8803) (width 0.2500) (layer "F.Cu") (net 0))
 (segment (start 141.1733 126.7500) (end 141.1733 126.7768) (width 0.2500) (layer "F.Cu") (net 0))
 (segment (start 141.1733 126.7768) (end 140.9879 126.9622) (width 0.2500) (layer "F.Cu") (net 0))
 (segment (start 140.9879 146.3017) (end 140.9879 126.9622) (width 0.2500) (layer "B.Cu") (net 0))
 (segment (start 120.7000 141.8500) (end 122.0267 141.8500) (width 0.2500) (layer "F.Cu") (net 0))
 (segment (start 122.0267 141.8500) (end 126.4784 146.3017) (width 0.2500) (layer "F.Cu") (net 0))
 (segment (start 126.4784 146.3017) (end 140.9879 146.3017) (width 0.2500) (layer "F.Cu") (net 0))
 (segment (start 142.2500 126.7500) (end 141.1733 126.7500) (width 0.2500) (layer "F.Cu") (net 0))
 (segment (start 148.8233 147.0000) (end 143.7608 141.9375) (width 0.2500) (layer "F.Cu") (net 6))
 (segment (start 143.7608 141.9375) (end 137.8313 141.9375) (width 0.2500) (layer "F.Cu") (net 6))
 (segment (start 150.0000 147.0000) (end 148.8233 147.0000) (width 0.2500) (layer "F.Cu") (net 6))
 (segment (start 137.9330 121.9903) (end 137.7500 122.1733) (width 0.2500) (layer "F.Cu") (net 6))
 (segment (start 137.8313 141.9375) (end 137.8313 122.0920) (width 0.2500) (layer "B.Cu") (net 6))
 (segment (start 137.8313 122.0920) (end 137.9330 121.9903) (width 0.2500) (layer "B.Cu") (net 6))
 (segment (start 137.7500 123.2500) (end 137.7500 122.1733) (width 0.2500) (layer "F.Cu") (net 6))
 (segment (start 133.7500 125.2500) (end 120.2750 125.2500) (width 0.2500) (layer "F.Cu") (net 7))
 (segment (start 120.2750 125.2500) (end 112.8250 117.8000) (width 0.2500) (layer "F.Cu") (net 7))
 (segment (start 112.8250 109.5000) (end 112.8250 117.8000) (width 0.2500) (layer "F.Cu") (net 7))
 (segment (start 112.0000 117.8000) (end 112.8250 117.8000) (width 0.2500) (layer "F.Cu") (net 7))
 (segment (start 132.8250 109.5000) (end 133.5517 109.5000) (width 0.2500) (layer "F.Cu") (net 8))
 (segment (start 139.7500 123.2500) (end 139.7500 115.6983) (width 0.2500) (layer "F.Cu") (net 8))
 (segment (start 139.7500 115.6983) (end 133.5517 109.5000) (width 0.2500) (layer "F.Cu") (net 8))
 (segment (start 135.7500 131.7500) (end 135.7500 132.9831) (width 0.2500) (layer "F.Cu") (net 9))
 (segment (start 135.7500 132.9831) (end 135.7311 133.0020) (width 0.2500) (layer "F.Cu") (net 9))
 (segment (start 135.7311 144.8281) (end 135.7311 133.0020) (width 0.2500) (layer "B.Cu") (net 9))
 (segment (start 133.5517 145.5000) (end 134.2236 144.8281) (width 0.2500) (layer "F.Cu") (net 9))
 (segment (start 134.2236 144.8281) (end 135.7311 144.8281) (width 0.2500) (layer "F.Cu") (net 9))
 (segment (start 132.8250 145.5000) (end 133.5517 145.5000) (width 0.2500) (layer "F.Cu") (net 9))
 (segment (start 161.6733 143.6000) (end 157.1964 139.1231) (width 0.2500) (layer "F.Cu") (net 10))
 (segment (start 157.1964 139.1231) (end 153.6242 139.1231) (width 0.2500) (layer "F.Cu") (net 10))
 (segment (start 153.6242 139.1231) (end 153.6227 139.1216) (width 0.2500) (layer "F.Cu") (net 10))
 (segment (start 153.6227 139.1216) (end 136.4312 139.1216) (width 0.2500) (layer "F.Cu") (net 10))
 (segment (start 137.2500 123.2500) (end 137.2500 122.1733) (width 0.2500) (layer "F.Cu") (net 10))
 (segment (start 137.2500 122.1733) (end 136.6325 122.1733) (width 0.2500) (layer "F.Cu") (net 10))
 (segment (start 136.6325 122.1733) (end 136.4312 121.9720) (width 0.2500) (layer "F.Cu") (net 10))
 (segment (start 136.4312 139.1216) (end 136.4312 121.9720) (width 0.2500) (layer "B.Cu") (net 10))
 (segment (start 162.8500 143.6000) (end 161.6733 143.6000) (width 0.2500) (layer "F.Cu") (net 10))
 (segment (start 169.1500 143.6000) (end 162.8500 143.6000) (width 0.2500) (layer "F.Cu") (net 10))
 (segment (start 143.3267 130.2500) (end 143.3314 130.2453) (width 0.2500) (layer "F.Cu") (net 11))
 (segment (start 143.3314 130.2453) (end 147.7375 130.2453) (width 0.2500) (layer "F.Cu") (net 11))
 (segment (start 147.7375 111.5783) (end 147.7375 130.2453) (width 0.2500) (layer "B.Cu") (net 11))
 (segment (start 159.3700 111.5783) (end 147.7375 111.5783) (width 0.2500) (layer "F.Cu") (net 11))
 (segment (start 159.3700 113.0300) (end 159.3700 111.5783) (width 0.2500) (layer "F.Cu") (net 11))
 (segment (start 142.2500 130.2500) (end 143.3267 130.2500) (width 0.2500) (layer "F.Cu") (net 11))
 (segment (start 142.2500 129.7500) (end 147.1020 129.7500) (width 0.2500) (layer "F.Cu") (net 12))
 (segment (start 147.1020 129.7500) (end 147.2877 129.5643) (width 0.2500) (layer "F.Cu") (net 12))
 (segment (start 147.2877 129.5643) (end 148.3770 129.5643) (width 0.2500) (layer "F.Cu") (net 12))
 (segment (start 148.3770 104.5183) (end 148.3770 129.5643) (width 0.2500) (layer "B.Cu") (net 12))
 (segment (start 160.6300 104.5183) (end 148.3770 104.5183) (width 0.2500) (layer "F.Cu") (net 12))
 (segment (start 160.6300 105.9700) (end 160.6300 104.5183) (width 0.2500) (layer "F.Cu") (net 12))
 (segment (start 158.0900 114.4817) (end 154.8414 114.4817) (width 0.2500) (layer "F.Cu") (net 13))
 (segment (start 154.8414 114.4817) (end 145.5838 123.7393) (width 0.2500) (layer "F.Cu") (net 13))
 (segment (start 145.5838 123.7393) (end 145.5838 127.5519) (width 0.2500) (layer "F.Cu") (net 13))
 (segment (start 145.5838 127.5519) (end 143.8857 129.2500) (width 0.2500) (layer "F.Cu") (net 13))
 (segment (start 143.8857 129.2500) (end 143.3267 129.2500) (width 0.2500) (layer "F.Cu") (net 13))
 (segment (start 158.0900 113.0300) (end 158.0900 114.4817) (width 0.2500) (layer "F.Cu") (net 13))
 (segment (start 142.2500 129.2500) (end 143.3267 129.2500) (width 0.2500) (layer "F.Cu") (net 13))
 (segment (start 161.9000 105.9700) (end 161.9000 104.5183) (width 0.2500) (layer "F.Cu") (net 14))
 (segment (start 161.9000 104.5183) (end 160.8935 103.5118) (width 0.2500) (layer "F.Cu") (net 14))
 (segment (start 160.8935 103.5118) (end 143.9816 103.5118) (width 0.2500) (layer "F.Cu") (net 14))
 (segment (start 143.9816 128.2411) (end 143.9816 103.5118) (width 0.2500) (layer "B.Cu") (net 14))
 (segment (start 143.9816 128.2411) (end 143.4727 128.7500) (width 0.2500) (layer "F.Cu") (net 14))
 (segment (start 143.4727 128.7500) (end 142.2500 128.7500) (width 0.2500) (layer "F.Cu") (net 14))
 (via (at 134.4039 136.2163) (size 0.6) (drill 0.3) (layers "F.Cu" "B.Cu") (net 2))
 (via (at 157.1910 134.5517) (size 0.6) (drill 0.3) (layers "F.Cu" "B.Cu") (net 2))
 (via (at 157.1910 126.3867) (size 0.6) (drill 0.3) (layers "F.Cu" "B.Cu") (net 2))
 (via (at 135.7021 128.3850) (size 0.6) (drill 0.3) (layers "F.Cu" "B.Cu") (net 2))
 (via (at 133.4767 121.5000) (size 0.6) (drill 0.3) (layers "F.Cu" "B.Cu") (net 2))
 (via (at 139.4570 127.7883) (size 0.6) (drill 0.3) (layers "F.Cu" "B.Cu") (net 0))
 (via (at 139.4570 147.8803) (size 0.6) (drill 0.3) (layers "F.Cu" "B.Cu") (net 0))
 (via (at 140.9879 126.9622) (size 0.6) (drill 0.3) (layers "F.Cu" "B.Cu") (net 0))
 (via (at 140.9879 146.3017) (size 0.6) (drill 0.3) (layers "F.Cu" "B.Cu") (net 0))
 (via (at 137.9330 121.9903) (size 0.6) (drill 0.3) (layers "F.Cu" "B.Cu") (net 6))
 (via (at 137.8313 141.9375) (size 0.6) (drill 0.3) (layers "F.Cu" "B.Cu") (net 6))
 (via (at 135.7311 144.8281) (size 0.6) (drill 0.3) (layers "F.Cu" "B.Cu") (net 9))
 (via (at 135.7311 133.0020) (size 0.6) (drill 0.3) (layers "F.Cu" "B.Cu") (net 9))
 (via (at 136.4312 139.1216) (size 0.6) (drill 0.3) (layers "F.Cu" "B.Cu") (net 10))
 (via (at 136.4312 121.9720) (size 0.6) (drill 0.3) (layers "F.Cu" "B.Cu") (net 10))
 (via (at 147.7375 130.2453) (size 0.6) (drill 0.3) (layers "F.Cu" "B.Cu") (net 11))
 (via (at 147.7375 111.5783) (size 0.6) (drill 0.3) (layers "F.Cu" "B.Cu") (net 11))
 (via (at 148.3770 129.5643) (size 0.6) (drill 0.3) (layers "F.Cu" "B.Cu") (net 12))
 (via (at 148.3770 104.5183) (size 0.6) (drill 0.3) (layers "F.Cu" "B.Cu") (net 12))
 (via (at 143.9816 128.2411) (size 0.6) (drill 0.3) (layers "F.Cu" "B.Cu") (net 14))
 (via (at 143.9816 103.5118) (size 0.6) (drill 0.3) (layers "F.Cu" "B.Cu") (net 14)))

